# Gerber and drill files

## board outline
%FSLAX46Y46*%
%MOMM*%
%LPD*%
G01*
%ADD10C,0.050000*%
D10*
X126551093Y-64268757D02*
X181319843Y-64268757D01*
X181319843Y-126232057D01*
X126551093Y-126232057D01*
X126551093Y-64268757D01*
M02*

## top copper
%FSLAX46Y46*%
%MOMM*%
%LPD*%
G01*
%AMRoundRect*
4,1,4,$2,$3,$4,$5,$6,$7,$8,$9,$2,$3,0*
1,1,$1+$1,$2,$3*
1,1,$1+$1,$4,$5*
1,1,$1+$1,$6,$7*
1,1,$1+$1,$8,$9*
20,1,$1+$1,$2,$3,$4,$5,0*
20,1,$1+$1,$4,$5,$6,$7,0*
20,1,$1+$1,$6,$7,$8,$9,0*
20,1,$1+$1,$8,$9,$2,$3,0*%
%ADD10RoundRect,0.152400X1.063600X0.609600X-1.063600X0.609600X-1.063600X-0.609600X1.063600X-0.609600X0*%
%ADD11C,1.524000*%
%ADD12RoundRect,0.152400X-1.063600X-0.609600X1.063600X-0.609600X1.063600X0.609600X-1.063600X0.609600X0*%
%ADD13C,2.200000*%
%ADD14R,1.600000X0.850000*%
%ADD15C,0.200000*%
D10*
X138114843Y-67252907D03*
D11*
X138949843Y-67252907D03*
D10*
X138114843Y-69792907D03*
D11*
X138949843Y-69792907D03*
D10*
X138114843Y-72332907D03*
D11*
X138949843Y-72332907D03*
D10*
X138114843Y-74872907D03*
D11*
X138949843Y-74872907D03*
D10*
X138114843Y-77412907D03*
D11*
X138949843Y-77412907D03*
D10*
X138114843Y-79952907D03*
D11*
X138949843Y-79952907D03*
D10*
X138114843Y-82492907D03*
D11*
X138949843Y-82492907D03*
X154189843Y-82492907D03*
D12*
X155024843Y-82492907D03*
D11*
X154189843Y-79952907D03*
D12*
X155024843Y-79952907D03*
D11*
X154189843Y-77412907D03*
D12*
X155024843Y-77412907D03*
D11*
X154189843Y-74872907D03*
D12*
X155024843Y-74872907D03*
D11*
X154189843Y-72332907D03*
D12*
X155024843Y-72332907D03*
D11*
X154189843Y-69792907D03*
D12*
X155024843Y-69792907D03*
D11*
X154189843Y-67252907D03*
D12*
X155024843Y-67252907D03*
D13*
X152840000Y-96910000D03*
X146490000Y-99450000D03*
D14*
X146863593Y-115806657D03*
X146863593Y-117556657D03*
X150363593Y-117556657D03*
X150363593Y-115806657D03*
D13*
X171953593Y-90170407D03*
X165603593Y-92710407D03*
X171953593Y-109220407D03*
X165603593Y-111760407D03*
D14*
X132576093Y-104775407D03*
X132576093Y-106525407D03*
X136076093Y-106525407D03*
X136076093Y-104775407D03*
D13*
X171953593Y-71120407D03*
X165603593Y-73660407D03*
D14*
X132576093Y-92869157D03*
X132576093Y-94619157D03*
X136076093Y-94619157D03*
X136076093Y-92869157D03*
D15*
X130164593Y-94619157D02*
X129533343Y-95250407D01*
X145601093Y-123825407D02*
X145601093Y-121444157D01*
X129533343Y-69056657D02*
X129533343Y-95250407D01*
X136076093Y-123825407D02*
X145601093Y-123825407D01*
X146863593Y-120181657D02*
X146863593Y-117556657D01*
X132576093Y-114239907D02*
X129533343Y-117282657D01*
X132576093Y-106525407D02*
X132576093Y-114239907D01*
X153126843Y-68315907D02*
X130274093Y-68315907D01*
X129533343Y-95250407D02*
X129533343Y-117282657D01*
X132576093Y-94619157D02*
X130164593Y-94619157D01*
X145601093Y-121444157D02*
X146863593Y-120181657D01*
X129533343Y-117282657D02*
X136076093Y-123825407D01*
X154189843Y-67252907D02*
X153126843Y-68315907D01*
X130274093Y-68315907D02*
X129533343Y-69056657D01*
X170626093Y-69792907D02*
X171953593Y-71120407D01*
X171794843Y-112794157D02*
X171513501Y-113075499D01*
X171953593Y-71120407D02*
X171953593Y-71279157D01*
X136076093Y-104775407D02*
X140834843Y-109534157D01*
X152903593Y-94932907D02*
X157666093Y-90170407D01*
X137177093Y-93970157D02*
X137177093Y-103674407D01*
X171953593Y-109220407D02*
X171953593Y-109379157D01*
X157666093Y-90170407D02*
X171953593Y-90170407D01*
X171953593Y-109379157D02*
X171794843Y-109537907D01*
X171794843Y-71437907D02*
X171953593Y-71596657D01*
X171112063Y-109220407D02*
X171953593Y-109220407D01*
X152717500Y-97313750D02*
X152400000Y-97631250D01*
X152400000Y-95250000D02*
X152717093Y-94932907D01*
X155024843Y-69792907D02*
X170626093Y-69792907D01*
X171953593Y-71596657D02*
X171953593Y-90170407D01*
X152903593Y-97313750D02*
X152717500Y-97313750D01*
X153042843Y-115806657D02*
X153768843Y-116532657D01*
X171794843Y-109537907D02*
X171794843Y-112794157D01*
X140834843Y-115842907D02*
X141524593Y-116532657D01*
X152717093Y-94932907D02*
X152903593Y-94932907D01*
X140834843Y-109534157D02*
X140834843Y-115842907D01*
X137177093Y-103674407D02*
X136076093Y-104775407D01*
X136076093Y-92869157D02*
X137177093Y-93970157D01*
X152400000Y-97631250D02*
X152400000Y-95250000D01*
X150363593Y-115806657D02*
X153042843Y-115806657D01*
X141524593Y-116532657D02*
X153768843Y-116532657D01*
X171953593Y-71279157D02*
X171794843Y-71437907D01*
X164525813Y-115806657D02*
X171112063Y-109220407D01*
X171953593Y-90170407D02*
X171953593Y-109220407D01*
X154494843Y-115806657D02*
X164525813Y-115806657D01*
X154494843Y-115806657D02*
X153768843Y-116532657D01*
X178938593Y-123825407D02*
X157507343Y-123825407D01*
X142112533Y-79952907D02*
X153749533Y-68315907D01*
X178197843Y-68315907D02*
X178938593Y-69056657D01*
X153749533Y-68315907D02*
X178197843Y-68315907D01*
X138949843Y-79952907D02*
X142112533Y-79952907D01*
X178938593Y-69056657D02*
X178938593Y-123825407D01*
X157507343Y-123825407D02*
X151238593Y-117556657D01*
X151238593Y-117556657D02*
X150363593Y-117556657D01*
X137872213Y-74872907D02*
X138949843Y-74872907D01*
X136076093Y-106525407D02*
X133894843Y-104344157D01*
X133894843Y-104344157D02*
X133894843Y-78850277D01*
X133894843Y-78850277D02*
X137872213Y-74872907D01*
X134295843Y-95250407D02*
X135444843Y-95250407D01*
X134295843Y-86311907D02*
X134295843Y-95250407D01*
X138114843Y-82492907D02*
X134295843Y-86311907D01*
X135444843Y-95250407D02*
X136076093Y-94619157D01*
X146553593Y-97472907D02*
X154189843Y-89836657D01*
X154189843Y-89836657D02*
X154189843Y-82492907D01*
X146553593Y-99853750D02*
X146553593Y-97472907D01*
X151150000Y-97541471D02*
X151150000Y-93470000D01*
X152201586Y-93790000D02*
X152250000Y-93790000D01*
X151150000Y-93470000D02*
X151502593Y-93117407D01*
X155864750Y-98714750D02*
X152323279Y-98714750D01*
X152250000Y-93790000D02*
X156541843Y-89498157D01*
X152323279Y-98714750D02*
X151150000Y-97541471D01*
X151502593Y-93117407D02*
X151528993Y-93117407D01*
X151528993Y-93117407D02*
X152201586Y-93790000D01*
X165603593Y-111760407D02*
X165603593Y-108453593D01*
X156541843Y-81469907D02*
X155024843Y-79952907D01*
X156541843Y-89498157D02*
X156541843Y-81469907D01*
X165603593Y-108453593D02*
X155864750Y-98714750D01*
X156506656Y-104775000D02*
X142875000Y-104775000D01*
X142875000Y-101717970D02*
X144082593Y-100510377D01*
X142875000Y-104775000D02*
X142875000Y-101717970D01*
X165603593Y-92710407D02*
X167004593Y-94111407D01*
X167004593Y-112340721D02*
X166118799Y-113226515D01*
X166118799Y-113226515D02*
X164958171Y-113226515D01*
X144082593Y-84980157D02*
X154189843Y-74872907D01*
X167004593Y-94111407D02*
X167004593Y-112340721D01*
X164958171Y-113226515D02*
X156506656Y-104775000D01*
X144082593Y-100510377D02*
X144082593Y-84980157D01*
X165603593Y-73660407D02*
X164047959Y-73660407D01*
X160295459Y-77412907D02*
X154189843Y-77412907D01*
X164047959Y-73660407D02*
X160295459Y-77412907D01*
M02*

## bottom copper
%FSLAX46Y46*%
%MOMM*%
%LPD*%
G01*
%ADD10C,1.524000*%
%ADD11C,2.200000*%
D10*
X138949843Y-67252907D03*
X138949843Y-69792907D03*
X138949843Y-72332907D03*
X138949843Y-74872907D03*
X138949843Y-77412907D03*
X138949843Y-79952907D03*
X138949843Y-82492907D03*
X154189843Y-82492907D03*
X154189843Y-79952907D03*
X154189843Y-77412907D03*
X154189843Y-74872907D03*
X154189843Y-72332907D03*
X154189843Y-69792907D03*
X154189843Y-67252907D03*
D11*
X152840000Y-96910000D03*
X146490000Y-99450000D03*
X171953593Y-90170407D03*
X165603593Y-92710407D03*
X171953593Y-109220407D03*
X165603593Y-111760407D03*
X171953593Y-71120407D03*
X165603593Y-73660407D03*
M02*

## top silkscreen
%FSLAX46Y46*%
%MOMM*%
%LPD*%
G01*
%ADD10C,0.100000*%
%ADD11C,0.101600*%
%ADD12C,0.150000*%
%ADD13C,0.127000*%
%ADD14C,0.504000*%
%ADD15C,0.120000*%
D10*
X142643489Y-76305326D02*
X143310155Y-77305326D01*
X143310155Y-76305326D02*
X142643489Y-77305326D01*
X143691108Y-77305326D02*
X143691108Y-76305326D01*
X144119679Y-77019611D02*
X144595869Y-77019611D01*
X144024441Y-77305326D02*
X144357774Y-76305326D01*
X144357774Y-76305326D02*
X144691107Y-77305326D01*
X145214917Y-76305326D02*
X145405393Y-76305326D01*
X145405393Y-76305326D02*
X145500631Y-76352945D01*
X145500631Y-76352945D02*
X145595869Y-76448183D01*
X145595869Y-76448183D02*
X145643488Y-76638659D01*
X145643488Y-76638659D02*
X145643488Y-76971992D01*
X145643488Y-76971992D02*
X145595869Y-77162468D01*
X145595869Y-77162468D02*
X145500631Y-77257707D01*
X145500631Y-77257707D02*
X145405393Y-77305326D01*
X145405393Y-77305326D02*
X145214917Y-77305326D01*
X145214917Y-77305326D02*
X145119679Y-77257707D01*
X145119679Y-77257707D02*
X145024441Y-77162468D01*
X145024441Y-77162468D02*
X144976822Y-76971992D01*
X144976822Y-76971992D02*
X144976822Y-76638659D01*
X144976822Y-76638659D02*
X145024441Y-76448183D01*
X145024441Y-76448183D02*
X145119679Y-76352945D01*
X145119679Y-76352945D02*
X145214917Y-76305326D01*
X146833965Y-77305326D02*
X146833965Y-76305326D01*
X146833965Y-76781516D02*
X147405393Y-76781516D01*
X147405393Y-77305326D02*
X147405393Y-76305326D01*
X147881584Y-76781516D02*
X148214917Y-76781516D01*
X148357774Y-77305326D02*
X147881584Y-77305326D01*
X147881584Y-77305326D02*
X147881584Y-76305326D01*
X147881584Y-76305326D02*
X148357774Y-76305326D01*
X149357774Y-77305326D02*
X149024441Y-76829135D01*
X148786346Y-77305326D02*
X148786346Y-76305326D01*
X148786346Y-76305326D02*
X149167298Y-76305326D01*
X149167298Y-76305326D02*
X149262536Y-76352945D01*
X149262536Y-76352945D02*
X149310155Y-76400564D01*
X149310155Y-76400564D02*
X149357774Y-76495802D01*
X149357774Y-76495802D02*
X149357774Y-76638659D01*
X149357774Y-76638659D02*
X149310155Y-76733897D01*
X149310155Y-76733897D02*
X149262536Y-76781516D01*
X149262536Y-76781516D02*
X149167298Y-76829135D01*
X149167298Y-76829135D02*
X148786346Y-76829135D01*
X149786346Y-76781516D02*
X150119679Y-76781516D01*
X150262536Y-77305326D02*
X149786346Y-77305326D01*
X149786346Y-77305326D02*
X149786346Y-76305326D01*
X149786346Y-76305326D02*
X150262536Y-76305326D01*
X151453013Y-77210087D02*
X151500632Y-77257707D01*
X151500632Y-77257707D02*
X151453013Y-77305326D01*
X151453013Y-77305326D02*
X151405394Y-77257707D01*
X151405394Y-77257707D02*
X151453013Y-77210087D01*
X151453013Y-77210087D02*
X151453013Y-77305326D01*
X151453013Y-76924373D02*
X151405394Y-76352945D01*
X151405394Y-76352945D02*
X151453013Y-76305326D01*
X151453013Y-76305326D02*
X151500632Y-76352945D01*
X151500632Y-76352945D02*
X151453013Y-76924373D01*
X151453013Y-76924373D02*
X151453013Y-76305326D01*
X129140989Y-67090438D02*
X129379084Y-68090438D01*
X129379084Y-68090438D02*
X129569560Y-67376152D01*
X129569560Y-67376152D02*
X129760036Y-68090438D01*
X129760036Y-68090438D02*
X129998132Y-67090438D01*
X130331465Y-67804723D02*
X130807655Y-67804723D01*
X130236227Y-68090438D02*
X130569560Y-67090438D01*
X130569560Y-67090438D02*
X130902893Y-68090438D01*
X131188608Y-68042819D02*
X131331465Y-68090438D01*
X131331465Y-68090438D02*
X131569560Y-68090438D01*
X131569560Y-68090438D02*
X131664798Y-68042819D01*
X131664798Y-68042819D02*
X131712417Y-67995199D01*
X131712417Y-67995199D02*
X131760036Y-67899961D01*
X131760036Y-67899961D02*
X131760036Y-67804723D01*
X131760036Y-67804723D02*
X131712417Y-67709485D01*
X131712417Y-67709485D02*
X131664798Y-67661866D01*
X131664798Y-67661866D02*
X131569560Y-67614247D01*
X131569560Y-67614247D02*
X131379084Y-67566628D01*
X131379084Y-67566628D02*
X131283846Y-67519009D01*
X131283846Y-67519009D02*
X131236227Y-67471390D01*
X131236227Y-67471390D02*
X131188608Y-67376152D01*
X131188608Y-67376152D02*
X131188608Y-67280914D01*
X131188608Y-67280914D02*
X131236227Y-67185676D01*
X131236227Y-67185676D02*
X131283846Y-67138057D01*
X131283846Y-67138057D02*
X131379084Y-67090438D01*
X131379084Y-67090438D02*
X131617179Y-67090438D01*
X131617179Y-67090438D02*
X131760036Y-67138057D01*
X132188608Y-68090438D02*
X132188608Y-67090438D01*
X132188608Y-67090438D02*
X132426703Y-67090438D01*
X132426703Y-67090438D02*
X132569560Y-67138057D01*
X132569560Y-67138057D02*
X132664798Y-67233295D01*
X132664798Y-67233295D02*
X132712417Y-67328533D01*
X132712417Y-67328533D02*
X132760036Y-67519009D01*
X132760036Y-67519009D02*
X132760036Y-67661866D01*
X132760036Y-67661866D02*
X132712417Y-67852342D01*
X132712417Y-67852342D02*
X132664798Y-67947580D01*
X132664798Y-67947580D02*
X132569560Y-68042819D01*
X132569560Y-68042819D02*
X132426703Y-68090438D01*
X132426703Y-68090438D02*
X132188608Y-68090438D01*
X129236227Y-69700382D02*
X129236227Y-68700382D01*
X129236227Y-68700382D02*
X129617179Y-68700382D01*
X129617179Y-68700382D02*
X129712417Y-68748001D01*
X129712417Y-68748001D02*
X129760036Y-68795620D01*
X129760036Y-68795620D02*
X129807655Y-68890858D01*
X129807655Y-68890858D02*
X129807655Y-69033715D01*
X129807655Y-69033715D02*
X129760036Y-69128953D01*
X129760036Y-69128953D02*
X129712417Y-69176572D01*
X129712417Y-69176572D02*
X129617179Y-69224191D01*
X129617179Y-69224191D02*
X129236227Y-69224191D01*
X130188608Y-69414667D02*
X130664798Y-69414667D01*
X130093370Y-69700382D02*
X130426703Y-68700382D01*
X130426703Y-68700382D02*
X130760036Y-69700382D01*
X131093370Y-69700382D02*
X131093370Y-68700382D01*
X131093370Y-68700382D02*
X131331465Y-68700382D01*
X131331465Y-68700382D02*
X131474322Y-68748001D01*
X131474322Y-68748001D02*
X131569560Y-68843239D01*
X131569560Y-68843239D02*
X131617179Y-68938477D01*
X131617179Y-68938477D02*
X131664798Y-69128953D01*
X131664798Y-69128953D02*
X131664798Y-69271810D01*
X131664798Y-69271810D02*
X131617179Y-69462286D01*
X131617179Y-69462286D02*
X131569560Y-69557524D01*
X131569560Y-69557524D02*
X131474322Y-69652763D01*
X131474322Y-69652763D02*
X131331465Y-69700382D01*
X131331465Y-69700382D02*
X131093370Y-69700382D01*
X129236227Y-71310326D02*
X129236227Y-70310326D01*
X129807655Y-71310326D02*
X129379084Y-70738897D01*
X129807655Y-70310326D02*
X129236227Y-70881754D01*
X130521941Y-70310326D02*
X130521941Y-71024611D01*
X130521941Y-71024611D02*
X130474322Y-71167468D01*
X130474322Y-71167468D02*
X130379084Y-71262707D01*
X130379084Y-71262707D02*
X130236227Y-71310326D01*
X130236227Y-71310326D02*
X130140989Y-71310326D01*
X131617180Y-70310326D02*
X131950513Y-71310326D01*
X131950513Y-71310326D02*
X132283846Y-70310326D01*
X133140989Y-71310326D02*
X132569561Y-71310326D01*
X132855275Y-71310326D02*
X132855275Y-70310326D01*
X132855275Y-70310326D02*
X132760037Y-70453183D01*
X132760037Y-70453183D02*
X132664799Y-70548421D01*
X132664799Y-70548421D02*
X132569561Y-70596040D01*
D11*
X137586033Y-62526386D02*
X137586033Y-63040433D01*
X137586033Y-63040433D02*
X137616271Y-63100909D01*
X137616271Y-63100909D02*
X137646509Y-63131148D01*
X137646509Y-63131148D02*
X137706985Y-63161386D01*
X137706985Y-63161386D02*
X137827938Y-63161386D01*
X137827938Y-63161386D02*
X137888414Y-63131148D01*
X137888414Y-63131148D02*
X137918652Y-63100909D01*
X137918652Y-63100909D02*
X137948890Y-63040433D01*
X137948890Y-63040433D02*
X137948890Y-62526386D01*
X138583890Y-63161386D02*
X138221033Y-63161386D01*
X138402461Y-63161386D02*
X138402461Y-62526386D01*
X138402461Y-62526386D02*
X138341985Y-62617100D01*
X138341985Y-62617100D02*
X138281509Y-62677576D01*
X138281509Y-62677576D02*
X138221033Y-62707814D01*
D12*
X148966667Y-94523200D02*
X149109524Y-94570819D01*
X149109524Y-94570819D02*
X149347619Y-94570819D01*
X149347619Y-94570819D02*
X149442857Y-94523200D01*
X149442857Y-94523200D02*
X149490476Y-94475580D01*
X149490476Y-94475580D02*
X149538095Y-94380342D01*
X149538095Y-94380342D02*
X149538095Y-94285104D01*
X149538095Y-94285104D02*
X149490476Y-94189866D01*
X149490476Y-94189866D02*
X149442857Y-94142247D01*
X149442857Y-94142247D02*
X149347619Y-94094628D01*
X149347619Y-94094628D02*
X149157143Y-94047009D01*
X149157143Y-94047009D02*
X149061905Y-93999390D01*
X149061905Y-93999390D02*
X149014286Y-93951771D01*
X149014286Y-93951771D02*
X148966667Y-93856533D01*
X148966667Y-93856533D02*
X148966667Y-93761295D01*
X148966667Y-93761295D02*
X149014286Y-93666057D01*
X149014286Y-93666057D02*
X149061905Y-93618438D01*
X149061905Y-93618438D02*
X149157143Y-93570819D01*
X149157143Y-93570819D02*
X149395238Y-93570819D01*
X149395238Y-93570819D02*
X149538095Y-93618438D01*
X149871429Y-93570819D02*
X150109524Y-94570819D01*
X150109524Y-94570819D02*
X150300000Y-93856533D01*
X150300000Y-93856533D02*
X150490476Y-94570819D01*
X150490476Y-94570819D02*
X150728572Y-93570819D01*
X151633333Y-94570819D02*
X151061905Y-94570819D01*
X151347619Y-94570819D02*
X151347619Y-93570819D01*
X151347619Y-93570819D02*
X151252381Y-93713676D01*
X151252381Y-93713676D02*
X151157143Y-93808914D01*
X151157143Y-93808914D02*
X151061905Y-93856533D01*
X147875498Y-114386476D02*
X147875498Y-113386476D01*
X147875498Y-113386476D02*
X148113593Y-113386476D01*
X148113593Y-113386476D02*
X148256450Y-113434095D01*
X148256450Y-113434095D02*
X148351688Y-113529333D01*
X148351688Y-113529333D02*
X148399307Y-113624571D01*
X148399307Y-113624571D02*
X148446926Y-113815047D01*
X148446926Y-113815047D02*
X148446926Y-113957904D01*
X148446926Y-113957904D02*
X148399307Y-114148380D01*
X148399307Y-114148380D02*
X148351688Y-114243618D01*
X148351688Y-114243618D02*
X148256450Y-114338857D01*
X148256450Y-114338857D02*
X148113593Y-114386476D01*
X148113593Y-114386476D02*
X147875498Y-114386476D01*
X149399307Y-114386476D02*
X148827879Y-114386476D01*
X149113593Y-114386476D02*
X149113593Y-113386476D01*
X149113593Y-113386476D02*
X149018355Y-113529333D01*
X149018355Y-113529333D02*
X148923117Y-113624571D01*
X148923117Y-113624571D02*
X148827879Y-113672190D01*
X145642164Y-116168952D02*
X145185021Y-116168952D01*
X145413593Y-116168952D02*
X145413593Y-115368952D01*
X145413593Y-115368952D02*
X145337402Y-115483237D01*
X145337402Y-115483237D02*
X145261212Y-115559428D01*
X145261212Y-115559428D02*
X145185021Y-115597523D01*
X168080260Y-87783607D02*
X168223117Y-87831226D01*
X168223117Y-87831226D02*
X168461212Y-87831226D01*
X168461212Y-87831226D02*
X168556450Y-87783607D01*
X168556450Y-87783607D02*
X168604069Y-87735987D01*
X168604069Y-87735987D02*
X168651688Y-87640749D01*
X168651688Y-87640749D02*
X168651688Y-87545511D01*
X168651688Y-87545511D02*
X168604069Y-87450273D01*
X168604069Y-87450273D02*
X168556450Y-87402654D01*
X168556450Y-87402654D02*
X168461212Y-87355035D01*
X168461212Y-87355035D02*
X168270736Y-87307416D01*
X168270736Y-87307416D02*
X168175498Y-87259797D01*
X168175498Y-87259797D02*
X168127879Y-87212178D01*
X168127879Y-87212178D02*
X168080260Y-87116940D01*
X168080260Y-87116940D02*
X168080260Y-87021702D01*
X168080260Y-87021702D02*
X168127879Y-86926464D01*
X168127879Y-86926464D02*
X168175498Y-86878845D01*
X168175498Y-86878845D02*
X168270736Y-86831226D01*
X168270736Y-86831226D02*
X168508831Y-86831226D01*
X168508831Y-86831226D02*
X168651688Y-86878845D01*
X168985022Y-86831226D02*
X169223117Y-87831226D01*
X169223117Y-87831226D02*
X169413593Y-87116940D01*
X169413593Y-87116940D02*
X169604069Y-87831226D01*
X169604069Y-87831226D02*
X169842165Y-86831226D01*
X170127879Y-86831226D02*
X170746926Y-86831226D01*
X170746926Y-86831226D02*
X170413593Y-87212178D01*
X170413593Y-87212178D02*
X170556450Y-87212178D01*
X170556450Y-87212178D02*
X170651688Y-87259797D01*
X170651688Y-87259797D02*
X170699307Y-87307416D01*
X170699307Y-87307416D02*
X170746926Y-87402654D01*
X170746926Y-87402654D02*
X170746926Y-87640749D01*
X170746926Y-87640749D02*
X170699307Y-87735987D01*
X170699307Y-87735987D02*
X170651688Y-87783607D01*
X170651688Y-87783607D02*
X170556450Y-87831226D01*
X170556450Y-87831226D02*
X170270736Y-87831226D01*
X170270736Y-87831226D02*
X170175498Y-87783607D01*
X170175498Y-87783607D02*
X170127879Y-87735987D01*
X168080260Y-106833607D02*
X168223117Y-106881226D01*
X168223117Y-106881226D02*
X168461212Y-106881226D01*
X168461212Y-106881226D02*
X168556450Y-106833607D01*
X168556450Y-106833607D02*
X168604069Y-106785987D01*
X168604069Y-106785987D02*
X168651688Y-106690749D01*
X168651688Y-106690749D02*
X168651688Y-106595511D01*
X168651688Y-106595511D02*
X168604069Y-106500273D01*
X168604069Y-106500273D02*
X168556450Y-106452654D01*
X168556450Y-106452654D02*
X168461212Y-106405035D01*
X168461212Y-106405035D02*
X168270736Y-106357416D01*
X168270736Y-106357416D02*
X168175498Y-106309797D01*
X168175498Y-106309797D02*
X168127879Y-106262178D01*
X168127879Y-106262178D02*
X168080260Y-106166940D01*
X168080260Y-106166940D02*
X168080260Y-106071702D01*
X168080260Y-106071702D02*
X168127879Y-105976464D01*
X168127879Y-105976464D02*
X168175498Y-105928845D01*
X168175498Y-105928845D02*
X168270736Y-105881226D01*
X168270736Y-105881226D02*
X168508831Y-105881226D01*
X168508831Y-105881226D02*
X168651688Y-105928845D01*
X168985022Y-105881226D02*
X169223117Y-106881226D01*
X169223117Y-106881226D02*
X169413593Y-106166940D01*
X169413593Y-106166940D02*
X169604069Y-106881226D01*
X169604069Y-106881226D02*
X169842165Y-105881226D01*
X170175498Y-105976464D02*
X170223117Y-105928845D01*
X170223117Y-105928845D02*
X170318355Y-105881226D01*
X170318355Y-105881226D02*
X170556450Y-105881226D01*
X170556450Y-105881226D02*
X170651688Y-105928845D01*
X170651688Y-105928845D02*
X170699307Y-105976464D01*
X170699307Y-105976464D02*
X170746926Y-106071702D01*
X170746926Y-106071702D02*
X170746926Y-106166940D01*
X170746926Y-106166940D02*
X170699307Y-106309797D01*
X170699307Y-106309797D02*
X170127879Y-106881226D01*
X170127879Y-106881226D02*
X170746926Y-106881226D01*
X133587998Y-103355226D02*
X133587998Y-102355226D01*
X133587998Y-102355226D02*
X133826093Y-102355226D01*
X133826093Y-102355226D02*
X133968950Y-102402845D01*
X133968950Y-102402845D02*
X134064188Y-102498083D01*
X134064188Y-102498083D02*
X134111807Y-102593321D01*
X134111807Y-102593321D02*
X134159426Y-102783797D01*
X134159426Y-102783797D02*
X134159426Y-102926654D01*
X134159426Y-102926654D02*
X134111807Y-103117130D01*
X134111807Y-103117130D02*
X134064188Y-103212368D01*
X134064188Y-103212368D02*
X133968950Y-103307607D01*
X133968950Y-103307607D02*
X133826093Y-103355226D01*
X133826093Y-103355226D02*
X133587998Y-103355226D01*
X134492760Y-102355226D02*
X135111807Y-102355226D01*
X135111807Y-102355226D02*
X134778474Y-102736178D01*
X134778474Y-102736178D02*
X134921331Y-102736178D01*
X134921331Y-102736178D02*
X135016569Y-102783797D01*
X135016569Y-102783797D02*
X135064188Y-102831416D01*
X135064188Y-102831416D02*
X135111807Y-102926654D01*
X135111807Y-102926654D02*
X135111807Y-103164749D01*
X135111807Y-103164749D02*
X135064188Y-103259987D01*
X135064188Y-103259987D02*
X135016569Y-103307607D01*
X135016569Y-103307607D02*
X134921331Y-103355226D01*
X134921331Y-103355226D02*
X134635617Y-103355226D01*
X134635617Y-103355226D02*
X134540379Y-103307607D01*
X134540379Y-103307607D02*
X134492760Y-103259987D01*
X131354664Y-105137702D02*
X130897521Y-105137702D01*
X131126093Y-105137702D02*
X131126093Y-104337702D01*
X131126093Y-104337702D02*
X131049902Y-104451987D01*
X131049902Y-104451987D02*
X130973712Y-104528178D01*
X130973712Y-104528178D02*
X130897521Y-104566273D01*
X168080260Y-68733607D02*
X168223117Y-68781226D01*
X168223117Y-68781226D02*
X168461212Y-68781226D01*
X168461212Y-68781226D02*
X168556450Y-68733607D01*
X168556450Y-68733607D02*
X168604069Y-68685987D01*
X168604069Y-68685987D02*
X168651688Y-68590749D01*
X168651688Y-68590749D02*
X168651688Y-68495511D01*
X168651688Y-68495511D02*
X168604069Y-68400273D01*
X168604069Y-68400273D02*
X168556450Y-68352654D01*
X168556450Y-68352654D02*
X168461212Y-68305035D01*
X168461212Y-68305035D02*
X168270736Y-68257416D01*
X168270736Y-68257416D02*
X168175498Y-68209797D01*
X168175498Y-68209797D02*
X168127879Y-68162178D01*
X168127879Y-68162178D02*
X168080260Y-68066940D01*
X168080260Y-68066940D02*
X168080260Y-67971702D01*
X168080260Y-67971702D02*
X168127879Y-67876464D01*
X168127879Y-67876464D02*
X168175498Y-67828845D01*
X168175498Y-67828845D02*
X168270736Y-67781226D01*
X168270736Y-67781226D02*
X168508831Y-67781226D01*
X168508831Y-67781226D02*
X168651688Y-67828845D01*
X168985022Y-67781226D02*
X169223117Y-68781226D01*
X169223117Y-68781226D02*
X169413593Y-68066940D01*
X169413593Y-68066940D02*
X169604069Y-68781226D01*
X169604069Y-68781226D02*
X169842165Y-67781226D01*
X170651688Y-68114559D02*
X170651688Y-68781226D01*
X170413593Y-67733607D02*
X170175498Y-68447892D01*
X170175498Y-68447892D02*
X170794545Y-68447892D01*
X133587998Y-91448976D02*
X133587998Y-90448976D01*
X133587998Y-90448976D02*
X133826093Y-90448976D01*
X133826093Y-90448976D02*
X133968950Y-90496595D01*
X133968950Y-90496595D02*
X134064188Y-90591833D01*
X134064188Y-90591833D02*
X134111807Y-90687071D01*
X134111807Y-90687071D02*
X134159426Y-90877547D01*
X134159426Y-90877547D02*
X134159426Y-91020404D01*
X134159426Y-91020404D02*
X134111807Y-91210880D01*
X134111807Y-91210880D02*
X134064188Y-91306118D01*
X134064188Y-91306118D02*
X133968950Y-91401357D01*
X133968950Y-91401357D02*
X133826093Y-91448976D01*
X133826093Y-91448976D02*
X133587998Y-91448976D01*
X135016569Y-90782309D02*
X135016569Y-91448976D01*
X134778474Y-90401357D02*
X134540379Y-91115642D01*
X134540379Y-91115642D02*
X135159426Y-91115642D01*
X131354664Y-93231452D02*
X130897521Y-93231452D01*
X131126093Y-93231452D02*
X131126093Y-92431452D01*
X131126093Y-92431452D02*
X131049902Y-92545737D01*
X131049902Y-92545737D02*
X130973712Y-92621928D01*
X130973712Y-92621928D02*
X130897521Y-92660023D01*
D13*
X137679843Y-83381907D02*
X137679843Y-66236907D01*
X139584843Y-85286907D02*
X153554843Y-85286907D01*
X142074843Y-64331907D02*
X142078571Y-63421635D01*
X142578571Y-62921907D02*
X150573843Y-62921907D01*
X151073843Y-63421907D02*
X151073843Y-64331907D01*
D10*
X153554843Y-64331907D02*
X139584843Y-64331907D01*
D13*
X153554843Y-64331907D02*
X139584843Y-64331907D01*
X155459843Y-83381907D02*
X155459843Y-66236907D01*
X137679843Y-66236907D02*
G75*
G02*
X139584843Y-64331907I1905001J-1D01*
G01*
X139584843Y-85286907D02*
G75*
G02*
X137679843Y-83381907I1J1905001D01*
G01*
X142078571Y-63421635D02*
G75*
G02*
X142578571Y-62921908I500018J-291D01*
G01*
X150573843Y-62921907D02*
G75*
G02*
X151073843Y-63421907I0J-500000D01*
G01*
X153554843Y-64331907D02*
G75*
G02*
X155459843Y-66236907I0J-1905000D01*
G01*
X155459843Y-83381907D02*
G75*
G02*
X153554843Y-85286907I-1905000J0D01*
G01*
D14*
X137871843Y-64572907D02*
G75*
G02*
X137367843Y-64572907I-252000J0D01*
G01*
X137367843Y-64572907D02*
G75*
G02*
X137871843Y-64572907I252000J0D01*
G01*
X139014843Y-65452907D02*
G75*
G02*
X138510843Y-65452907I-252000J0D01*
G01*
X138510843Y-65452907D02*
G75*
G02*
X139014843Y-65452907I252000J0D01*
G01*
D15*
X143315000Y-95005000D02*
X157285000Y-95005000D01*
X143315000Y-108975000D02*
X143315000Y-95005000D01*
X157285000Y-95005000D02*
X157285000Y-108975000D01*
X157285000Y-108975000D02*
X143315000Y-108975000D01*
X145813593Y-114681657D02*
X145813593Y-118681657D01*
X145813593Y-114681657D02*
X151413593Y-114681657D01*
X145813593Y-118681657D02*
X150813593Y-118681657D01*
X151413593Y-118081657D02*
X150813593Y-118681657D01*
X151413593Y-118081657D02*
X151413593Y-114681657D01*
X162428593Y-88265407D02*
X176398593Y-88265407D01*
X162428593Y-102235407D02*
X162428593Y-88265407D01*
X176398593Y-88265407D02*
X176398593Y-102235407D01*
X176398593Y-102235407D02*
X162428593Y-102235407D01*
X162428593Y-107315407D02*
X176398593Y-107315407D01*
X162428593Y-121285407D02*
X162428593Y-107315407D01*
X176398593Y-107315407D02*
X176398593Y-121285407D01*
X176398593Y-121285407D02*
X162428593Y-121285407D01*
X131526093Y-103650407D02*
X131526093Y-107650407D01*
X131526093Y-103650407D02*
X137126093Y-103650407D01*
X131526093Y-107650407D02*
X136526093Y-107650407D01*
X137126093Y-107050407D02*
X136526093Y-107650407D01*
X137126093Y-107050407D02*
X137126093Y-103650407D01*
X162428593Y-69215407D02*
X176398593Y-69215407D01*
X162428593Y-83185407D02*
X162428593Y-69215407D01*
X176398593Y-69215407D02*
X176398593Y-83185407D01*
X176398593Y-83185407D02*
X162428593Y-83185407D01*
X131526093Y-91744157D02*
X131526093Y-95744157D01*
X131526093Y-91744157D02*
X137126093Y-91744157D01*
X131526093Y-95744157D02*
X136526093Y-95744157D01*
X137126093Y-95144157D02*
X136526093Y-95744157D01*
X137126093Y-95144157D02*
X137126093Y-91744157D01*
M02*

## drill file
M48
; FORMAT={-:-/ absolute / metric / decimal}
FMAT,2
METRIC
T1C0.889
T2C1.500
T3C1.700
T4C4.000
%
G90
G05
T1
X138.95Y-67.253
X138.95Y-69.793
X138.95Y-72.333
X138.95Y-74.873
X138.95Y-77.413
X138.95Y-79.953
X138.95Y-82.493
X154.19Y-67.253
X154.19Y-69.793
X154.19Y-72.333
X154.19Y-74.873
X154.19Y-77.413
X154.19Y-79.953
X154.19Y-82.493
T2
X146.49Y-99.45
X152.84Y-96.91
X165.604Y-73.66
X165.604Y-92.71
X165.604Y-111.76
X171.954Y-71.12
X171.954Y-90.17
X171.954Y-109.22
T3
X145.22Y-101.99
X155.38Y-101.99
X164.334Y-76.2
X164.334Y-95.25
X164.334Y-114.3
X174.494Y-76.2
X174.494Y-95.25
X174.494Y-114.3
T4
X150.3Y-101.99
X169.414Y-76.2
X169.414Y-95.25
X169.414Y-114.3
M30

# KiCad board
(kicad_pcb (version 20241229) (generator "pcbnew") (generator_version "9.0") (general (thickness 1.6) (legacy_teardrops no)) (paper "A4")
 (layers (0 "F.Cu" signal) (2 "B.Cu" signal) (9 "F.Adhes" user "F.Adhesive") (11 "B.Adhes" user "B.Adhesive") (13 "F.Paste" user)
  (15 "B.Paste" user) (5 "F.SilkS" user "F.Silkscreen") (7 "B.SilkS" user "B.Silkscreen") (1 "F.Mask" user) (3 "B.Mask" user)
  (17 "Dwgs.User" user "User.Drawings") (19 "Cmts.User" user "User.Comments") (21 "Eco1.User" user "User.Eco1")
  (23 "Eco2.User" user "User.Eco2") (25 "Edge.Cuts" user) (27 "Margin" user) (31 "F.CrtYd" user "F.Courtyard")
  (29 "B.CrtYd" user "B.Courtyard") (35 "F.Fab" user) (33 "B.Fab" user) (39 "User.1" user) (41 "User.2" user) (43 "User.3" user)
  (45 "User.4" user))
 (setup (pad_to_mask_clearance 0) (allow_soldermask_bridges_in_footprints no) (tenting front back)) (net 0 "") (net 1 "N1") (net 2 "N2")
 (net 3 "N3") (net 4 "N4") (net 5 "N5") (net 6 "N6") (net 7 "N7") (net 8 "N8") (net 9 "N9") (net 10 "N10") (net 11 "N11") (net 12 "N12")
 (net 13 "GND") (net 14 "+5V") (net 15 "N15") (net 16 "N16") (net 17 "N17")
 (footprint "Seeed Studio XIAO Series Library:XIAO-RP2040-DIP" (layer "F.Cu") (at 146.569843 74.872907)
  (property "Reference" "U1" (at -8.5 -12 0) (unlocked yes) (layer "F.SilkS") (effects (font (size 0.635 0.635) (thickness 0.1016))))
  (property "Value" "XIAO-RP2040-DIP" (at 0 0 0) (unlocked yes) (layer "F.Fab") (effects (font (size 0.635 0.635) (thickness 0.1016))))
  (fp_line (start -8.89 8.509) (end -8.89 -8.636) (stroke (width 0.127) (type solid)) (layer "F.SilkS"))
  (fp_line (start -6.985 10.414) (end 6.985 10.414) (stroke (width 0.127) (type solid)) (layer "F.SilkS"))
  (fp_line (start -4.495 -10.541) (end -4.491272 -11.451272) (stroke (width 0.127) (type solid)) (layer "F.SilkS"))
  (fp_line (start -3.991272 -11.951) (end 4.004 -11.951) (stroke (width 0.127) (type solid)) (layer "F.SilkS"))
  (fp_line (start 4.504 -11.451) (end 4.504 -10.541) (stroke (width 0.127) (type solid)) (layer "F.SilkS"))
  (fp_line (start 6.985 -10.541) (end -6.985 -10.541) (stroke (width 0.1) (type solid)) (layer "F.SilkS"))
  (fp_line (start 6.985 -10.541) (end -6.985 -10.541) (stroke (width 0.127) (type solid)) (layer "F.SilkS"))
  (fp_line (start 8.89 8.509) (end 8.89 -8.636) (stroke (width 0.127) (type solid)) (layer "F.SilkS"))
  (fp_arc (start -8.89 -8.636) (mid -8.332038 -9.983038) (end -6.985 -10.541) (stroke (width 0.127) (type solid)) (layer "F.SilkS"))
  (fp_arc (start -6.985 10.414) (mid -8.332038 9.856038) (end -8.89 8.509) (stroke (width 0.127) (type solid)) (layer "F.SilkS"))
  (fp_arc (start -4.491272 -11.451272) (mid -4.344728 -11.80464) (end -3.991272 -11.951) (stroke (width 0.127) (type default))
   (layer "F.SilkS"))
  (fp_arc (start 4.004 -11.951) (mid 4.357553 -11.804553) (end 4.504 -11.451) (stroke (width 0.127) (type default)) (layer "F.SilkS"))
  (fp_arc (start 6.985 -10.541) (mid 8.332038 -9.983038) (end 8.89 -8.636) (stroke (width 0.127) (type solid)) (layer "F.SilkS"))
  (fp_arc (start 8.89 8.509) (mid 8.332038 9.856038) (end 6.985 10.414) (stroke (width 0.127) (type solid)) (layer "F.SilkS"))
  (fp_circle (center -8.95 -10.3) (end -8.95 -10.554) (stroke (width 0.5) (type solid)) (fill yes) (layer "F.SilkS"))
  (fp_circle (center -7.807 -9.42) (end -7.807 -9.674) (stroke (width 0.5) (type solid)) (fill yes) (layer "F.SilkS"))
  (pad "1" smd roundrect (at -8.455 -7.62 180) (size 2.432 1.524) (layers "F.Cu" "F.Mask") (roundrect_rratio 0.1) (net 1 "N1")
   (thermal_bridge_angle 45))
  (pad "1" thru_hole circle (at -7.62 -7.62 180) (size 1.524 1.524) (drill 0.889) (layers "*.Cu" "*.Mask") (remove_unused_layers no)
   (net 1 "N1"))
  (pad "2" smd roundrect (at -8.455 -5.08 180) (size 2.432 1.524) (layers "F.Cu" "F.Mask") (roundrect_rratio 0.1) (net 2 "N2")
   (thermal_bridge_angle 45))
  (pad "2" thru_hole circle (at -7.62 -5.08 180) (size 1.524 1.524) (drill 0.889) (layers "*.Cu" "*.Mask") (remove_unused_layers no)
   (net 2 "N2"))
  (pad "3" smd roundrect (at -8.455 -2.54 180) (size 2.432 1.524) (layers "F.Cu" "F.Mask") (roundrect_rratio 0.1) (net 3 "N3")
   (thermal_bridge_angle 45))
  (pad "3" thru_hole circle (at -7.62 -2.54 180) (size 1.524 1.524) (drill 0.889) (layers "*.Cu" "*.Mask") (remove_unused_layers no)
   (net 3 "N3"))
  (pad "4" smd roundrect (at -8.455 0 180) (size 2.432 1.524) (layers "F.Cu" "F.Mask") (roundrect_rratio 0.1) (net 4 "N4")
   (thermal_bridge_angle 45))
  (pad "4" thru_hole circle (at -7.62 0 180) (size 1.524 1.524) (drill 0.889) (layers "*.Cu" "*.Mask") (remove_unused_layers no)
   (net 4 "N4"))
  (pad "5" smd roundrect (at -8.455 2.54 180) (size 2.432 1.524) (layers "F.Cu" "F.Mask") (roundrect_rratio 0.1) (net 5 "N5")
   (thermal_bridge_angle 45))
  (pad "5" thru_hole circle (at -7.62 2.54 180) (size 1.524 1.524) (drill 0.889) (layers "*.Cu" "*.Mask") (remove_unused_layers no)
   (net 5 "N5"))
  (pad "6" smd roundrect (at -8.455 5.08 180) (size 2.432 1.524) (layers "F.Cu" "F.Mask") (roundrect_rratio 0.1) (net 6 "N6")
   (thermal_bridge_angle 45))
  (pad "6" thru_hole circle (at -7.62 5.08 180) (size 1.524 1.524) (drill 0.889) (layers "*.Cu" "*.Mask") (remove_unused_layers no)
   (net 6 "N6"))
  (pad "7" smd roundrect (at -8.455 7.62 180) (size 2.432 1.524) (layers "F.Cu" "F.Mask") (roundrect_rratio 0.1) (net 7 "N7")
   (thermal_bridge_angle 45))
  (pad "7" thru_hole circle (at -7.62 7.62 180) (size 1.524 1.524) (drill 0.889) (layers "*.Cu" "*.Mask") (remove_unused_layers no)
   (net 7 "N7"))
  (pad "8" thru_hole circle (at 7.62 7.62) (size 1.524 1.524) (drill 0.889) (layers "*.Cu" "*.Mask") (remove_unused_layers no) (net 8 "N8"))
  (pad "8" smd roundrect (at 8.455 7.62) (size 2.432 1.524) (layers "F.Cu" "F.Mask") (roundrect_rratio 0.1) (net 8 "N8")
   (thermal_bridge_angle 45))
  (pad "9" thru_hole circle (at 7.62 5.08) (size 1.524 1.524) (drill 0.889) (layers "*.Cu" "*.Mask") (remove_unused_layers no) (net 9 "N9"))
  (pad "9" smd roundrect (at 8.455 5.08) (size 2.432 1.524) (layers "F.Cu" "F.Mask") (roundrect_rratio 0.1) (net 9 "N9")
   (thermal_bridge_angle 45))
  (pad "10" thru_hole circle (at 7.62 2.54) (size 1.524 1.524) (drill 0.889) (layers "*.Cu" "*.Mask") (remove_unused_layers no)
   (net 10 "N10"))
  (pad "10" smd roundrect (at 8.455 2.54) (size 2.432 1.524) (layers "F.Cu" "F.Mask") (roundrect_rratio 0.1) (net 10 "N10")
   (thermal_bridge_angle 45))
  (pad "11" thru_hole circle (at 7.62 0) (size 1.524 1.524) (drill 0.889) (layers "*.Cu" "*.Mask") (remove_unused_layers no) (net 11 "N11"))
  (pad "11" smd roundrect (at 8.455 0) (size 2.432 1.524) (layers "F.Cu" "F.Mask") (roundrect_rratio 0.1) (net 11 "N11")
   (thermal_bridge_angle 45))
  (pad "12" thru_hole circle (at 7.62 -2.54) (size 1.524 1.524) (drill 0.889) (layers "*.Cu" "*.Mask") (remove_unused_layers no)
   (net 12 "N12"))
  (pad "12" smd roundrect (at 8.455 -2.54) (size 2.432 1.524) (layers "F.Cu" "F.Mask") (roundrect_rratio 0.1) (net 12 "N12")
   (thermal_bridge_angle 45))
  (pad "13" thru_hole circle (at 7.62 -5.08) (size 1.524 1.524) (drill 0.889) (layers "*.Cu" "*.Mask") (remove_unused_layers no)
   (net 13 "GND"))
  (pad "13" smd roundrect (at 8.455 -5.08) (size 2.432 1.524) (layers "F.Cu" "F.Mask") (roundrect_rratio 0.1) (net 13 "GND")
   (thermal_bridge_angle 45))
  (pad "14" thru_hole circle (at 7.62 -7.62) (size 1.524 1.524) (drill 0.889) (layers "*.Cu" "*.Mask") (remove_unused_layers no)
   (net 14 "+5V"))
  (pad "14" smd roundrect (at 8.455 -7.62) (size 2.432 1.524) (layers "F.Cu" "F.Mask") (roundrect_rratio 0.1) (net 14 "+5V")
   (thermal_bridge_angle 45)))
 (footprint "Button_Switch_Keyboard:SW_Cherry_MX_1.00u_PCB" (layer "F.Cu") (at 152.84 96.91)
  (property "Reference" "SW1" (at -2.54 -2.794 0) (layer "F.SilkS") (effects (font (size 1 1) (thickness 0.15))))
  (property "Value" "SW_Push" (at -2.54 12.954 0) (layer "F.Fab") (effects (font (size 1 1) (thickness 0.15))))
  (fp_line (start -9.525 -1.905) (end 4.445 -1.905) (stroke (width 0.12) (type solid)) (layer "F.SilkS"))
  (fp_line (start -9.525 12.065) (end -9.525 -1.905) (stroke (width 0.12) (type solid)) (layer "F.SilkS"))
  (fp_line (start 4.445 -1.905) (end 4.445 12.065) (stroke (width 0.12) (type solid)) (layer "F.SilkS"))
  (fp_line (start 4.445 12.065) (end -9.525 12.065) (stroke (width 0.12) (type solid)) (layer "F.SilkS"))
  (pad "" np_thru_hole circle (at -7.62 5.08) (size 1.7 1.7) (drill 1.7) (layers "*.Cu" "*.Mask"))
  (pad "" np_thru_hole circle (at -2.54 5.08) (size 4 4) (drill 4) (layers "*.Cu" "*.Mask"))
  (pad "" np_thru_hole circle (at 2.54 5.08) (size 1.7 1.7) (drill 1.7) (layers "*.Cu" "*.Mask"))
  (pad "1" thru_hole circle (at 0 0) (size 2.2 2.2) (drill 1.5) (layers "*.Cu" "*.Mask") (remove_unused_layers no) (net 13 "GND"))
  (pad "2" thru_hole circle (at -6.35 2.54) (size 2.2 2.2) (drill 1.5) (layers "*.Cu" "*.Mask") (remove_unused_layers no) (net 8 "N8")))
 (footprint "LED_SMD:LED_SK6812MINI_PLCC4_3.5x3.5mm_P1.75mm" (layer "F.Cu") (at 148.613593 116.681657)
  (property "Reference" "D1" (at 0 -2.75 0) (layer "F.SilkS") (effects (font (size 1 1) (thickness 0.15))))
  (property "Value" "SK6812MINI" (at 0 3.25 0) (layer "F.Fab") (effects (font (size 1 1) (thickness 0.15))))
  (fp_line (start -2.8 -2) (end -2.8 2) (stroke (width 0.12) (type default)) (layer "F.SilkS"))
  (fp_line (start -2.8 -2) (end 2.8 -2) (stroke (width 0.12) (type solid)) (layer "F.SilkS"))
  (fp_line (start -2.8 2) (end 2.2 2) (stroke (width 0.12) (type solid)) (layer "F.SilkS"))
  (fp_line (start 2.8 1.4) (end 2.2 2) (stroke (width 0.12) (type default)) (layer "F.SilkS"))
  (fp_line (start 2.8 1.4) (end 2.8 -2) (stroke (width 0.12) (type solid)) (layer "F.SilkS"))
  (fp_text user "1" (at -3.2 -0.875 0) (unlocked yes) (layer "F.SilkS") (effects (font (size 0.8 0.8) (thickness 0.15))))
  (pad "1" smd rect (at -1.75 -0.875) (size 1.6 0.85) (layers "F.Cu" "F.Mask" "F.Paste") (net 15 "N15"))
  (pad "2" smd rect (at -1.75 0.875) (size 1.6 0.85) (layers "F.Cu" "F.Mask" "F.Paste") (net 14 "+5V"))
  (pad "3" smd rect (at 1.75 0.875) (size 1.6 0.85) (layers "F.Cu" "F.Mask" "F.Paste") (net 6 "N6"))
  (pad "4" smd rect (at 1.75 -0.875) (size 1.6 0.85) (layers "F.Cu" "F.Mask" "F.Paste") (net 13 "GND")))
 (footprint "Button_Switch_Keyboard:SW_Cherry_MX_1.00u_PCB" (layer "F.Cu") (at 171.953593 90.170407)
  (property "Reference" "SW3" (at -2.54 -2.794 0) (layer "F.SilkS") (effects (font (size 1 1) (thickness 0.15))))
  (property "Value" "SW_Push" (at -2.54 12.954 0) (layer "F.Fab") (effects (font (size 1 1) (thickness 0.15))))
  (fp_line (start -9.525 -1.905) (end 4.445 -1.905) (stroke (width 0.12) (type solid)) (layer "F.SilkS"))
  (fp_line (start -9.525 12.065) (end -9.525 -1.905) (stroke (width 0.12) (type solid)) (layer "F.SilkS"))
  (fp_line (start 4.445 -1.905) (end 4.445 12.065) (stroke (width 0.12) (type solid)) (layer "F.SilkS"))
  (fp_line (start 4.445 12.065) (end -9.525 12.065) (stroke (width 0.12) (type solid)) (layer "F.SilkS"))
  (pad "" np_thru_hole circle (at -7.62 5.08) (size 1.7 1.7) (drill 1.7) (layers "*.Cu" "*.Mask"))
  (pad "" np_thru_hole circle (at -2.54 5.08) (size 4 4) (drill 4) (layers "*.Cu" "*.Mask"))
  (pad "" np_thru_hole circle (at 2.54 5.08) (size 1.7 1.7) (drill 1.7) (layers "*.Cu" "*.Mask"))
  (pad "1" thru_hole circle (at 0 0) (size 2.2 2.2) (drill 1.5) (layers "*.Cu" "*.Mask") (remove_unused_layers no) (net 13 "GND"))
  (pad "2" thru_hole circle (at -6.35 2.54) (size 2.2 2.2) (drill 1.5) (layers "*.Cu" "*.Mask") (remove_unused_layers no) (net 11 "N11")))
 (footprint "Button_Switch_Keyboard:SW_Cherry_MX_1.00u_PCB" (layer "F.Cu") (at 171.953593 109.220407)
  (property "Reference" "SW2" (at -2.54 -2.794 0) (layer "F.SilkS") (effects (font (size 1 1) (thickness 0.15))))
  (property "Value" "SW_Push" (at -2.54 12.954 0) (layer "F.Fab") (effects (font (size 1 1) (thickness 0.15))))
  (fp_line (start -9.525 -1.905) (end 4.445 -1.905) (stroke (width 0.12) (type solid)) (layer "F.SilkS"))
  (fp_line (start -9.525 12.065) (end -9.525 -1.905) (stroke (width 0.12) (type solid)) (layer "F.SilkS"))
  (fp_line (start 4.445 -1.905) (end 4.445 12.065) (stroke (width 0.12) (type solid)) (layer "F.SilkS"))
  (fp_line (start 4.445 12.065) (end -9.525 12.065) (stroke (width 0.12) (type solid)) (layer "F.SilkS"))
  (pad "" np_thru_hole circle (at -7.62 5.08) (size 1.7 1.7) (drill 1.7) (layers "*.Cu" "*.Mask"))
  (pad "" np_thru_hole circle (at -2.54 5.08) (size 4 4) (drill 4) (layers "*.Cu" "*.Mask"))
  (pad "" np_thru_hole circle (at 2.54 5.08) (size 1.7 1.7) (drill 1.7) (layers "*.Cu" "*.Mask"))
  (pad "1" thru_hole circle (at 0 0) (size 2.2 2.2) (drill 1.5) (layers "*.Cu" "*.Mask") (remove_unused_layers no) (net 13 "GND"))
  (pad "2" thru_hole circle (at -6.35 2.54) (size 2.2 2.2) (drill 1.5) (layers "*.Cu" "*.Mask") (remove_unused_layers no) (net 9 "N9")))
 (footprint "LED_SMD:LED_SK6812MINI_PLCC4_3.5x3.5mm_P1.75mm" (layer "F.Cu") (at 134.326093 105.650407)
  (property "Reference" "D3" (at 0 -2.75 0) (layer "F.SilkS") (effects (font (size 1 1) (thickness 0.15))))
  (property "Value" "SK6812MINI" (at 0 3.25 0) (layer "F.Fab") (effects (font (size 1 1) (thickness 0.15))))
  (fp_line (start -2.8 -2) (end -2.8 2) (stroke (width 0.12) (type default)) (layer "F.SilkS"))
  (fp_line (start -2.8 -2) (end 2.8 -2) (stroke (width 0.12) (type solid)) (layer "F.SilkS"))
  (fp_line (start -2.8 2) (end 2.2 2) (stroke (width 0.12) (type solid)) (layer "F.SilkS"))
  (fp_line (start 2.8 1.4) (end 2.2 2) (stroke (width 0.12) (type default)) (layer "F.SilkS"))
  (fp_line (start 2.8 1.4) (end 2.8 -2) (stroke (width 0.12) (type solid)) (layer "F.SilkS"))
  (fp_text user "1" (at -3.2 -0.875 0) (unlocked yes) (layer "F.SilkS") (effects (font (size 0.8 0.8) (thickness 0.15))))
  (pad "1" smd rect (at -1.75 -0.875) (size 1.6 0.85) (layers "F.Cu" "F.Mask" "F.Paste") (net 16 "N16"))
  (pad "2" smd rect (at -1.75 0.875) (size 1.6 0.85) (layers "F.Cu" "F.Mask" "F.Paste") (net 14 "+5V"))
  (pad "3" smd rect (at 1.75 0.875) (size 1.6 0.85) (layers "F.Cu" "F.Mask" "F.Paste") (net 4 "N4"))
  (pad "4" smd rect (at 1.75 -0.875) (size 1.6 0.85) (layers "F.Cu" "F.Mask" "F.Paste") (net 13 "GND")))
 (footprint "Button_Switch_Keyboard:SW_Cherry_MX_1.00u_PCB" (layer "F.Cu") (at 171.953593 71.120407)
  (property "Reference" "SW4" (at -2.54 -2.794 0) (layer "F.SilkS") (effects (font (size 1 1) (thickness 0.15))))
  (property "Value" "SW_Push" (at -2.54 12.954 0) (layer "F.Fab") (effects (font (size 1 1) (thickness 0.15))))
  (fp_line (start -9.525 -1.905) (end 4.445 -1.905) (stroke (width 0.12) (type solid)) (layer "F.SilkS"))
  (fp_line (start -9.525 12.065) (end -9.525 -1.905) (stroke (width 0.12) (type solid)) (layer "F.SilkS"))
  (fp_line (start 4.445 -1.905) (end 4.445 12.065) (stroke (width 0.12) (type solid)) (layer "F.SilkS"))
  (fp_line (start 4.445 12.065) (end -9.525 12.065) (stroke (width 0.12) (type solid)) (layer "F.SilkS"))
  (pad "" np_thru_hole circle (at -7.62 5.08) (size 1.7 1.7) (drill 1.7) (layers "*.Cu" "*.Mask"))
  (pad "" np_thru_hole circle (at -2.54 5.08) (size 4 4) (drill 4) (layers "*.Cu" "*.Mask"))
  (pad "" np_thru_hole circle (at 2.54 5.08) (size 1.7 1.7) (drill 1.7) (layers "*.Cu" "*.Mask"))
  (pad "1" thru_hole circle (at 0 0) (size 2.2 2.2) (drill 1.5) (layers "*.Cu" "*.Mask") (remove_unused_layers no) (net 13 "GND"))
  (pad "2" thru_hole circle (at -6.35 2.54) (size 2.2 2.2) (drill 1.5) (layers "*.Cu" "*.Mask") (remove_unused_layers no) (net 10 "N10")))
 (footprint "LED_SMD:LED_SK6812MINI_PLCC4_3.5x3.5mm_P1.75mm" (layer "F.Cu") (at 134.326093 93.744157)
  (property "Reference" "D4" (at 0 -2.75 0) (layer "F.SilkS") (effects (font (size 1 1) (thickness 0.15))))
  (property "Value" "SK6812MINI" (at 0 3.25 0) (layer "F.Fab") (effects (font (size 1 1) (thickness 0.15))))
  (fp_line (start -2.8 -2) (end -2.8 2) (stroke (width 0.12) (type default)) (layer "F.SilkS"))
  (fp_line (start -2.8 -2) (end 2.8 -2) (stroke (width 0.12) (type solid)) (layer "F.SilkS"))
  (fp_line (start -2.8 2) (end 2.2 2) (stroke (width 0.12) (type solid)) (layer "F.SilkS"))
  (fp_line (start 2.8 1.4) (end 2.2 2) (stroke (width 0.12) (type default)) (layer "F.SilkS"))
  (fp_line (start 2.8 1.4) (end 2.8 -2) (stroke (width 0.12) (type solid)) (layer "F.SilkS"))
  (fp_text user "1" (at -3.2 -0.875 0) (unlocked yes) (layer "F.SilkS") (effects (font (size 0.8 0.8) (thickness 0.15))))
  (pad "1" smd rect (at -1.75 -0.875) (size 1.6 0.85) (layers "F.Cu" "F.Mask" "F.Paste") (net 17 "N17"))
  (pad "2" smd rect (at -1.75 0.875) (size 1.6 0.85) (layers "F.Cu" "F.Mask" "F.Paste") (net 14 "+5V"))
  (pad "3" smd rect (at 1.75 0.875) (size 1.6 0.85) (layers "F.Cu" "F.Mask" "F.Paste") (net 7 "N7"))
  (pad "4" smd rect (at 1.75 -0.875) (size 1.6 0.85) (layers "F.Cu" "F.Mask" "F.Paste") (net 13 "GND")))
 (gr_rect (start 126.551093 64.268757) (end 181.319843 126.232057) (stroke (width 0.05) (type default)) (fill no) (layer "Edge.Cuts"))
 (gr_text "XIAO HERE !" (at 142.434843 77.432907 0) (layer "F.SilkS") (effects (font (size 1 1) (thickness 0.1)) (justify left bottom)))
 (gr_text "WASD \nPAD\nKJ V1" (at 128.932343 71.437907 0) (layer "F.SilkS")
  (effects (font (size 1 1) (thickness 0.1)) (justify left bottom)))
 (segment (start 130.164593 94.619157) (end 129.533343 95.250407) (width 0.2) (layer "F.Cu") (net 14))
 (segment (start 145.601093 123.825407) (end 145.601093 121.444157) (width 0.2) (layer "F.Cu") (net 14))
 (segment (start 129.533343 69.056657) (end 129.533343 95.250407) (width 0.2) (layer "F.Cu") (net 14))
 (segment (start 136.076093 123.825407) (end 145.601093 123.825407) (width 0.2) (layer "F.Cu") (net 14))
 (segment (start 146.863593 120.181657) (end 146.863593 117.556657) (width 0.2) (layer "F.Cu") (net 14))
 (segment (start 132.576093 114.239907) (end 129.533343 117.282657) (width 0.2) (layer "F.Cu") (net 14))
 (segment (start 132.576093 106.525407) (end 132.576093 114.239907) (width 0.2) (layer "F.Cu") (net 14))
 (segment (start 153.126843 68.315907) (end 130.274093 68.315907) (width 0.2) (layer "F.Cu") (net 14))
 (segment (start 129.533343 95.250407) (end 129.533343 117.282657) (width 0.2) (layer "F.Cu") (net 14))
 (segment (start 132.576093 94.619157) (end 130.164593 94.619157) (width 0.2) (layer "F.Cu") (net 14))
 (segment (start 145.601093 121.444157) (end 146.863593 120.181657) (width 0.2) (layer "F.Cu") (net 14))
 (segment (start 129.533343 117.282657) (end 136.076093 123.825407) (width 0.2) (layer "F.Cu") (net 14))
 (segment (start 154.189843 67.252907) (end 153.126843 68.315907) (width 0.2) (layer "F.Cu") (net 14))
 (segment (start 130.274093 68.315907) (end 129.533343 69.056657) (width 0.2) (layer "F.Cu") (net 14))
 (segment (start 170.626093 69.792907) (end 171.953593 71.120407) (width 0.2) (layer "F.Cu") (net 13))
 (segment (start 171.794843 112.794157) (end 171.513501 113.075499) (width 0.2) (layer "F.Cu") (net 13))
 (segment (start 171.953593 71.120407) (end 171.953593 71.279157) (width 0.2) (layer "F.Cu") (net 13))
 (segment (start 136.076093 104.775407) (end 140.834843 109.534157) (width 0.2) (layer "F.Cu") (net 13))
 (segment (start 152.903593 94.932907) (end 157.666093 90.170407) (width 0.2) (layer "F.Cu") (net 13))
 (segment (start 137.177093 93.970157) (end 137.177093 103.674407) (width 0.2) (layer "F.Cu") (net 13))
 (segment (start 171.953593 109.220407) (end 171.953593 109.379157) (width 0.2) (layer "F.Cu") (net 13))
 (segment (start 157.666093 90.170407) (end 171.953593 90.170407) (width 0.2) (layer "F.Cu") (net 13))
 (segment (start 171.953593 109.379157) (end 171.794843 109.537907) (width 0.2) (layer "F.Cu") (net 13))
 (segment (start 171.794843 71.437907) (end 171.953593 71.596657) (width 0.2) (layer "F.Cu") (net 13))
 (segment (start 171.112063 109.220407) (end 171.953593 109.220407) (width 0.2) (layer "F.Cu") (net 13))
 (segment (start 152.7175 97.31375) (end 152.4 97.63125) (width 0.2) (layer "F.Cu") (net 13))
 (segment (start 152.4 95.25) (end 152.717093 94.932907) (width 0.2) (layer "F.Cu") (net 13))
 (segment (start 155.024843 69.792907) (end 170.626093 69.792907) (width 0.2) (layer "F.Cu") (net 13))
 (segment (start 171.953593 71.596657) (end 171.953593 90.170407) (width 0.2) (layer "F.Cu") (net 13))
 (segment (start 152.903593 97.31375) (end 152.7175 97.31375) (width 0.2) (layer "F.Cu") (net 13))
 (segment (start 153.042843 115.806657) (end 153.768843 116.532657) (width 0.2) (layer "F.Cu") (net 13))
 (segment (start 171.794843 109.537907) (end 171.794843 112.794157) (width 0.2) (layer "F.Cu") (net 13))
 (segment (start 140.834843 115.842907) (end 141.524593 116.532657) (width 0.2) (layer "F.Cu") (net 13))
 (segment (start 152.717093 94.932907) (end 152.903593 94.932907) (width 0.2) (layer "F.Cu") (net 13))
 (segment (start 140.834843 109.534157) (end 140.834843 115.842907) (width 0.2) (layer "F.Cu") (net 13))
 (segment (start 137.177093 103.674407) (end 136.076093 104.775407) (width 0.2) (layer "F.Cu") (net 13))
 (segment (start 136.076093 92.869157) (end 137.177093 93.970157) (width 0.2) (layer "F.Cu") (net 13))
 (segment (start 152.4 97.63125) (end 152.4 95.25) (width 0.2) (layer "F.Cu") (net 13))
 (segment (start 150.363593 115.806657) (end 153.042843 115.806657) (width 0.2) (layer "F.Cu") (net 13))
 (segment (start 141.524593 116.532657) (end 153.768843 116.532657) (width 0.2) (layer "F.Cu") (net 13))
 (segment (start 171.953593 71.279157) (end 171.794843 71.437907) (width 0.2) (layer "F.Cu") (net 13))
 (segment (start 164.525813 115.806657) (end 171.112063 109.220407) (width 0.2) (layer "F.Cu") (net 13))
 (segment (start 171.953593 90.170407) (end 171.953593 109.220407) (width 0.2) (layer "F.Cu") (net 13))
 (segment (start 154.494843 115.806657) (end 164.525813 115.806657) (width 0.2) (layer "F.Cu") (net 13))
 (segment (start 154.494843 115.806657) (end 153.768843 116.532657) (width 0.2) (layer "F.Cu") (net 13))
 (segment (start 178.938593 123.825407) (end 157.507343 123.825407) (width 0.2) (layer "F.Cu") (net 6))
 (segment (start 142.112533 79.952907) (end 153.749533 68.315907) (width 0.2) (layer "F.Cu") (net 6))
 (segment (start 178.197843 68.315907) (end 178.938593 69.056657) (width 0.2) (layer "F.Cu") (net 6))
 (segment (start 153.749533 68.315907) (end 178.197843 68.315907) (width 0.2) (layer "F.Cu") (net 6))
 (segment (start 138.949843 79.952907) (end 142.112533 79.952907) (width 0.2) (layer "F.Cu") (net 6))
 (segment (start 178.938593 69.056657) (end 178.938593 123.825407) (width 0.2) (layer "F.Cu") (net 6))
 (segment (start 157.507343 123.825407) (end 151.238593 117.556657) (width 0.2) (layer "F.Cu") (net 6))
 (segment (start 151.238593 117.556657) (end 150.363593 117.556657) (width 0.2) (layer "F.Cu") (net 6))
 (segment (start 137.872213 74.872907) (end 138.949843 74.872907) (width 0.2) (layer "F.Cu") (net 4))
 (segment (start 136.076093 106.525407) (end 133.894843 104.344157) (width 0.2) (layer "F.Cu") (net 4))
 (segment (start 133.894843 104.344157) (end 133.894843 78.850277) (width 0.2) (layer "F.Cu") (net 4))
 (segment (start 133.894843 78.850277) (end 137.872213 74.872907) (width 0.2) (layer "F.Cu") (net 4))
 (segment (start 134.295843 95.250407) (end 135.444843 95.250407) (width 0.2) (layer "F.Cu") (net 7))
 (segment (start 134.295843 86.311907) (end 134.295843 95.250407) (width 0.2) (layer "F.Cu") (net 7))
 (segment (start 138.114843 82.492907) (end 134.295843 86.311907) (width 0.2) (layer "F.Cu") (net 7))
 (segment (start 135.444843 95.250407) (end 136.076093 94.619157) (width 0.2) (layer "F.Cu") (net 7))
 (segment (start 146.553593 97.472907) (end 154.189843 89.836657) (width 0.2) (layer "F.Cu") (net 8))
 (segment (start 154.189843 89.836657) (end 154.189843 82.492907) (width 0.2) (layer "F.Cu") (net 8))
 (segment (start 146.553593 99.85375) (end 146.553593 97.472907) (width 0.2) (layer "F.Cu") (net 8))
 (segment (start 151.15 97.541471) (end 151.15 93.47) (width 0.2) (layer "F.Cu") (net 9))
 (segment (start 152.201586 93.79) (end 152.25 93.79) (width 0.2) (layer "F.Cu") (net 9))
 (segment (start 151.15 93.47) (end 151.502593 93.117407) (width 0.2) (layer "F.Cu") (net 9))
 (segment (start 155.86475 98.71475) (end 152.323279 98.71475) (width 0.2) (layer "F.Cu") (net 9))
 (segment (start 152.25 93.79) (end 156.541843 89.498157) (width 0.2) (layer "F.Cu") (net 9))
 (segment (start 152.323279 98.71475) (end 151.15 97.541471) (width 0.2) (layer "F.Cu") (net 9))
 (segment (start 151.502593 93.117407) (end 151.528993 93.117407) (width 0.2) (layer "F.Cu") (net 9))
 (segment (start 151.528993 93.117407) (end 152.201586 93.79) (width 0.2) (layer "F.Cu") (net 9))
 (segment (start 165.603593 111.760407) (end 165.603593 108.453593) (width 0.2) (layer "F.Cu") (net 9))
 (segment (start 156.541843 81.469907) (end 155.024843 79.952907) (width 0.2) (layer "F.Cu") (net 9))
 (segment (start 156.541843 89.498157) (end 156.541843 81.469907) (width 0.2) (layer "F.Cu") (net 9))
 (segment (start 165.603593 108.453593) (end 155.86475 98.71475) (width 0.2) (layer "F.Cu") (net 9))
 (segment (start 156.506656 104.775) (end 142.875 104.775) (width 0.2) (layer "F.Cu") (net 11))
 (segment (start 142.875 101.71797) (end 144.082593 100.510377) (width 0.2) (layer "F.Cu") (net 11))
 (segment (start 142.875 104.775) (end 142.875 101.71797) (width 0.2) (layer "F.Cu") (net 11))
 (segment (start 165.603593 92.710407) (end 167.004593 94.111407) (width 0.2) (layer "F.Cu") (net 11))
 (segment (start 167.004593 112.340721) (end 166.118799 113.226515) (width 0.2) (layer "F.Cu") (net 11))
 (segment (start 166.118799 113.226515) (end 164.958171 113.226515) (width 0.2) (layer "F.Cu") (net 11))
 (segment (start 144.082593 84.980157) (end 154.189843 74.872907) (width 0.2) (layer "F.Cu") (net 11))
 (segment (start 167.004593 94.111407) (end 167.004593 112.340721) (width 0.2) (layer "F.Cu") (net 11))
 (segment (start 164.958171 113.226515) (end 156.506656 104.775) (width 0.2) (layer "F.Cu") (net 11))
 (segment (start 144.082593 100.510377) (end 144.082593 84.980157) (width 0.2) (layer "F.Cu") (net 11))
 (segment (start 165.603593 73.660407) (end 164.047959 73.660407) (width 0.2) (layer "F.Cu") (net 10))
 (segment (start 160.295459 77.412907) (end 154.189843 77.412907) (width 0.2) (layer "F.Cu") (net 10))
 (segment (start 164.047959 73.660407) (end 160.295459 77.412907) (width 0.2) (layer "F.Cu") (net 10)))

